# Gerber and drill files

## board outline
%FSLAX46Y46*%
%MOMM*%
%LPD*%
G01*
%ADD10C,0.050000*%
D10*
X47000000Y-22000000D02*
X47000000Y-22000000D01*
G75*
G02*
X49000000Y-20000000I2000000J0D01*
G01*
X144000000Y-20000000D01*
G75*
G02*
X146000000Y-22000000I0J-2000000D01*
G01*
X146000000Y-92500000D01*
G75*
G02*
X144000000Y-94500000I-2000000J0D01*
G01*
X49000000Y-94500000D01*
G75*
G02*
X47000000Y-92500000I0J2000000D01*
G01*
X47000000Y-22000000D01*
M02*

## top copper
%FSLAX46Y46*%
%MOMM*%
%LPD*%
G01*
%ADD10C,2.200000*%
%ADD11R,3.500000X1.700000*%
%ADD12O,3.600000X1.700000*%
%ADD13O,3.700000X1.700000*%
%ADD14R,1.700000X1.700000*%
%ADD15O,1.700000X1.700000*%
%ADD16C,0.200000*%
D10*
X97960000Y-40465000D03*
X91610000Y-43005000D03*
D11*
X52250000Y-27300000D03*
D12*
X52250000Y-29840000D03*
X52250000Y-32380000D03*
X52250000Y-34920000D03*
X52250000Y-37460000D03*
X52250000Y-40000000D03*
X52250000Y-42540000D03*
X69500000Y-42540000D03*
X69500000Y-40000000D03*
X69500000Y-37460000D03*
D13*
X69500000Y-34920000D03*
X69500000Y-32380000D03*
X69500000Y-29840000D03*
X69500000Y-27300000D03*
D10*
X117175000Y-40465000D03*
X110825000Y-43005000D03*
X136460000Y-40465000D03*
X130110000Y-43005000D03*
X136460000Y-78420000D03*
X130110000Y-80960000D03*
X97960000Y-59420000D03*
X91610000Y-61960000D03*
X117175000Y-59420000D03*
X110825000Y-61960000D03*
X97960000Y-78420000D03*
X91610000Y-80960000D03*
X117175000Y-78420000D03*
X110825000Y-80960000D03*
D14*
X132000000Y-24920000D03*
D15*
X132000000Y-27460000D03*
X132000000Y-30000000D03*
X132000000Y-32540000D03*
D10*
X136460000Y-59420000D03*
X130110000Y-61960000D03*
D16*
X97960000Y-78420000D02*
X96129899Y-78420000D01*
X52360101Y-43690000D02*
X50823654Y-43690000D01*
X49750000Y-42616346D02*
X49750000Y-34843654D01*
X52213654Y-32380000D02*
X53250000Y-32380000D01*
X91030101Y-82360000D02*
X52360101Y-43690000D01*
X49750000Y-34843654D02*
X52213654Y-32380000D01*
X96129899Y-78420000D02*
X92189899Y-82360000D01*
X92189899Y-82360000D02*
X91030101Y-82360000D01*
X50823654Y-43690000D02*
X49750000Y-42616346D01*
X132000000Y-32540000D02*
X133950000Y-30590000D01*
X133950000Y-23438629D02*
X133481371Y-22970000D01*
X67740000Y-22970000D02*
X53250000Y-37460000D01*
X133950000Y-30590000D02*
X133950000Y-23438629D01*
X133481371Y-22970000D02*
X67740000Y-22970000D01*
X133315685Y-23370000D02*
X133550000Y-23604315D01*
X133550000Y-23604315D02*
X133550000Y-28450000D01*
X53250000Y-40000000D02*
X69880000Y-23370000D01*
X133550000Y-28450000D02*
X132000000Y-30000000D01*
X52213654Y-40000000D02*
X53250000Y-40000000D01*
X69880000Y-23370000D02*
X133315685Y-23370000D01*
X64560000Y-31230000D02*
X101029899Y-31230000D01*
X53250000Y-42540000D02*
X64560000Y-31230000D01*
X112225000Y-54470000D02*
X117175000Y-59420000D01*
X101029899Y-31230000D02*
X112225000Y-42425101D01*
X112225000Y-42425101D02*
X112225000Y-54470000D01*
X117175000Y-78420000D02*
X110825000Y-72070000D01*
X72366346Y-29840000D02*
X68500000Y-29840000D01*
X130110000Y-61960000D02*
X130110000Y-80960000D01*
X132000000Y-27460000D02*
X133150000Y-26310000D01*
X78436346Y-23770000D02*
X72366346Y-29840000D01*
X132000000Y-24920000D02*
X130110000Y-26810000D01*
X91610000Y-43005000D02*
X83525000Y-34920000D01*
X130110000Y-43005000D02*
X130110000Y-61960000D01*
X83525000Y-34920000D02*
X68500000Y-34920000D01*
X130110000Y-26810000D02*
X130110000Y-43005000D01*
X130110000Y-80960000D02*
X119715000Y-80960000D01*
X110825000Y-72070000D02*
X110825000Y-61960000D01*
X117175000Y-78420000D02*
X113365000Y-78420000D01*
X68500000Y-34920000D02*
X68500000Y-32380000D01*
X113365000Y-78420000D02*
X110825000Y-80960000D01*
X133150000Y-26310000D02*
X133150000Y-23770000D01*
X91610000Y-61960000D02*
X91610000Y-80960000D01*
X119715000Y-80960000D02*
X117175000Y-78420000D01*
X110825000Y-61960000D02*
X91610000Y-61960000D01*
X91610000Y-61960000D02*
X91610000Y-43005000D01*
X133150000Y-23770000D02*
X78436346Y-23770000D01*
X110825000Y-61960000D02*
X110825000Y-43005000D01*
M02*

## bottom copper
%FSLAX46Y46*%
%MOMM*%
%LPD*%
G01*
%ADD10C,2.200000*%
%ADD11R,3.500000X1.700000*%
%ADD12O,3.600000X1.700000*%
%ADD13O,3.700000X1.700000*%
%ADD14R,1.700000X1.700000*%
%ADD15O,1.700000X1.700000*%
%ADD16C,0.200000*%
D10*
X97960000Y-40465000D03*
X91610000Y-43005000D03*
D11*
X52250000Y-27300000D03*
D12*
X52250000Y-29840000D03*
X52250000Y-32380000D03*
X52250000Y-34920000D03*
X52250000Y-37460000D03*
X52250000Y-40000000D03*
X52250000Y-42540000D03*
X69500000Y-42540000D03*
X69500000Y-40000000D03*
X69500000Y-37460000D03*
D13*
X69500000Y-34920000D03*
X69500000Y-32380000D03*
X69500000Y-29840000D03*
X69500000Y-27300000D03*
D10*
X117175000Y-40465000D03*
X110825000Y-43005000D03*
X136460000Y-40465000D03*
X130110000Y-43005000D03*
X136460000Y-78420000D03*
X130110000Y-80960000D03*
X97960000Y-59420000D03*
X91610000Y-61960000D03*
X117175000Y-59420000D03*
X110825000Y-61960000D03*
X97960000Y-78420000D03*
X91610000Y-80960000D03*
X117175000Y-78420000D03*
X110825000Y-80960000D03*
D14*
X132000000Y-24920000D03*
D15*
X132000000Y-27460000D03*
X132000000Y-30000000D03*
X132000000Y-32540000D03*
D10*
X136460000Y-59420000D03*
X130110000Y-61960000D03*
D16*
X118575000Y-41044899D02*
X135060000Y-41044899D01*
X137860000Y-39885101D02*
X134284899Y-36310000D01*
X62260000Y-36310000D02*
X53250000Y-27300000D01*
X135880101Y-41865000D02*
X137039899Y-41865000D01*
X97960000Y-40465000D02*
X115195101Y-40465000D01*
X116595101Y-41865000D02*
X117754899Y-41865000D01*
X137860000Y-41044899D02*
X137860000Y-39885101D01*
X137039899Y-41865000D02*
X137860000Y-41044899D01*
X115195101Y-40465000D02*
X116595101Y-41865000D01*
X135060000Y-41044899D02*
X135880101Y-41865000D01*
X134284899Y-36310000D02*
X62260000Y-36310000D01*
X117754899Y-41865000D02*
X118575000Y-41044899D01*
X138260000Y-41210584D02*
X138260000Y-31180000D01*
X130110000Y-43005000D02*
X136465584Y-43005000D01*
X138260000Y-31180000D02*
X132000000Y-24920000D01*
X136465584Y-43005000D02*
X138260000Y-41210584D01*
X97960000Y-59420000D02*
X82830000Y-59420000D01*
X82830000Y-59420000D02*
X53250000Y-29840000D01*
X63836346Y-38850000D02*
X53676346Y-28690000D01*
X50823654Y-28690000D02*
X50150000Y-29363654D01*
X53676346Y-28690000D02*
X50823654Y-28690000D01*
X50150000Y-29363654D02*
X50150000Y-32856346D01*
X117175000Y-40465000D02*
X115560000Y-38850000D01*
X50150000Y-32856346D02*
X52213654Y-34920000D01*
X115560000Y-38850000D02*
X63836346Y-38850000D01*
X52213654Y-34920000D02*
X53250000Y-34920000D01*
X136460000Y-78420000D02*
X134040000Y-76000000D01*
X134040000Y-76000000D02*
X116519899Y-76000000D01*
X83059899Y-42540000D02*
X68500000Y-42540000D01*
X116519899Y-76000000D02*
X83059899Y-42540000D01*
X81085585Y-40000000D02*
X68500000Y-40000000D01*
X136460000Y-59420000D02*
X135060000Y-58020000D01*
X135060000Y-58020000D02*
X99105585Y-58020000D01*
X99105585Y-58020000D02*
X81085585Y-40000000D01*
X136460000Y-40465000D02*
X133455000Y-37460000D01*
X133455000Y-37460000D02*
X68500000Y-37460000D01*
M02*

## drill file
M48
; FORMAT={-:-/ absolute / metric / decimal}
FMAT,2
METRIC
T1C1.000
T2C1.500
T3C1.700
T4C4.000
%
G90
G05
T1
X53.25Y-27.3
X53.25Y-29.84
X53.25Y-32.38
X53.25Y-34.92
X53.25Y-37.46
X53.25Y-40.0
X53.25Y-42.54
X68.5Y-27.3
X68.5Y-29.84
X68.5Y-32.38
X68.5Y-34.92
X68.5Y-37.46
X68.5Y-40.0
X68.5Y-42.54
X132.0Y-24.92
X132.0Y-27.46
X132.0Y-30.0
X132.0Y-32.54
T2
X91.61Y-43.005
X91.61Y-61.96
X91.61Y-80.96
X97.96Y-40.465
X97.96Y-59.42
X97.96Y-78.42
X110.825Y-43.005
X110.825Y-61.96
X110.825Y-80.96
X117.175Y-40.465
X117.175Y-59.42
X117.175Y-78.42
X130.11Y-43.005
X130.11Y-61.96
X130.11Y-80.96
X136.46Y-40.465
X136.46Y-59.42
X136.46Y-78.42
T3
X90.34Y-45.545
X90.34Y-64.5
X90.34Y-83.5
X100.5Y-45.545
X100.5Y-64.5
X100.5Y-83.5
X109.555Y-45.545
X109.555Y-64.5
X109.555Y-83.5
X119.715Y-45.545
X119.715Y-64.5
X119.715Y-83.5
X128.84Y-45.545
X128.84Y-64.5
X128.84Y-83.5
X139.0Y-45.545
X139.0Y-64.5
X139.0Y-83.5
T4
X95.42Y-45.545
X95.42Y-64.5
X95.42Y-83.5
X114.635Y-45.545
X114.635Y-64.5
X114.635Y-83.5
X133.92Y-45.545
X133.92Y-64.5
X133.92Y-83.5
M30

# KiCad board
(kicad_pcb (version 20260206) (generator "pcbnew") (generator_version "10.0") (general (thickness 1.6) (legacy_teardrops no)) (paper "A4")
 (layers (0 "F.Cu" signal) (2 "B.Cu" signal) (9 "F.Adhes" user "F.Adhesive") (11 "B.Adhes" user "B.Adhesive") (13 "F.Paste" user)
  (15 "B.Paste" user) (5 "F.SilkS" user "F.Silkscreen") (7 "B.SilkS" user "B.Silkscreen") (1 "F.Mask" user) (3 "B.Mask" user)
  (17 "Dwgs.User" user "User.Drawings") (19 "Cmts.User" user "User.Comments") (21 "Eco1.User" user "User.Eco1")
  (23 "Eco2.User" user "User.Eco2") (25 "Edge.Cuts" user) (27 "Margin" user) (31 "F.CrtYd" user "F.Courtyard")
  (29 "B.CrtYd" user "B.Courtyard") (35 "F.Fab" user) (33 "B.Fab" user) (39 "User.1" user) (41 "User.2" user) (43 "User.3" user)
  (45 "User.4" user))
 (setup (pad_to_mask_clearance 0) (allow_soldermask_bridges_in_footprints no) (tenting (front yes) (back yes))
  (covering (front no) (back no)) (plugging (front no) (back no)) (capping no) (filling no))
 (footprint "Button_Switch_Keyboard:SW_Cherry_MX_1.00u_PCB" (layer "F.Cu") (at 97.96 40.465)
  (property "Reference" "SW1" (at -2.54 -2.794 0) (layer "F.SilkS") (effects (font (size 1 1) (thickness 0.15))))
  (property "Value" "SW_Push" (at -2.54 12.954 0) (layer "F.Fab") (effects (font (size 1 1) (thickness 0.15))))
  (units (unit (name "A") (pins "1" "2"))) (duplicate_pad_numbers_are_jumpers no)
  (pad "" np_thru_hole circle (at -7.62 5.08) (size 1.7 1.7) (drill 1.7) (layers "*.Cu" "*.Mask"))
  (pad "" np_thru_hole circle (at -2.54 5.08) (size 4 4) (drill 4) (layers "*.Cu" "*.Mask"))
  (pad "" np_thru_hole circle (at 2.54 5.08) (size 1.7 1.7) (drill 1.7) (layers "*.Cu" "*.Mask"))
  (pad "1" thru_hole circle (at 0 0) (size 2.2 2.2) (drill 1.5) (layers "*.Cu" "*.Mask") (remove_unused_layers no) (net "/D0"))
  (pad "2" thru_hole circle (at -6.35 2.54) (size 2.2 2.2) (drill 1.5) (layers "*.Cu" "*.Mask") (remove_unused_layers no) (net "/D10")))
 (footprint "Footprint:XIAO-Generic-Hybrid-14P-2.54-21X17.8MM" (layer "F.Cu") (at 60.875 34.92)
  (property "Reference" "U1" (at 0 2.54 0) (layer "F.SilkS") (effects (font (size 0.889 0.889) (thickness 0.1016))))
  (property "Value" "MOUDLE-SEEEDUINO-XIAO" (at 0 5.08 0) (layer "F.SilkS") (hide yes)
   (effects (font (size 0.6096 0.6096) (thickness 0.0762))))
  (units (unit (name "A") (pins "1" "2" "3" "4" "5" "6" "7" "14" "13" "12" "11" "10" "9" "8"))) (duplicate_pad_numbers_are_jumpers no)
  (pad "1" thru_hole rect (at -7.625 -7.62) (size 3.5 1.7) (drill 1 (offset -1 0)) (layers "*.Cu" "*.Mask") (remove_unused_layers no)
   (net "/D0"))
  (pad "2" thru_hole oval (at -7.625 -5.08) (size 3.6 1.7) (drill 1 (offset -1 0)) (layers "*.Cu" "*.Mask") (remove_unused_layers no)
   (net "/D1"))
  (pad "3" thru_hole oval (at -7.625 -2.54) (size 3.6 1.7) (drill 1 (offset -1 0)) (layers "*.Cu" "*.Mask") (remove_unused_layers no)
   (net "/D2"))
  (pad "4" thru_hole oval (at -7.625 0) (size 3.6 1.7) (drill 1 (offset -1 0)) (layers "*.Cu" "*.Mask") (remove_unused_layers no)
   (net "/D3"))
  (pad "5" thru_hole oval (at -7.625 2.54) (size 3.6 1.7) (drill 1 (offset -1 0)) (layers "*.Cu" "*.Mask") (remove_unused_layers no)
   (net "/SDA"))
  (pad "6" thru_hole oval (at -7.625 5.08 180) (size 3.6 1.7) (drill 1 (offset 1 0)) (layers "*.Cu" "*.Mask") (remove_unused_layers no)
   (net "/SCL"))
  (pad "7" thru_hole oval (at -7.625 7.62) (size 3.6 1.7) (drill 1 (offset -1 0)) (layers "*.Cu" "*.Mask") (remove_unused_layers no)
   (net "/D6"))
  (pad "8" thru_hole oval (at 7.625 7.62) (size 3.6 1.7) (drill 1 (offset 1 0)) (layers "*.Cu" "*.Mask") (remove_unused_layers no)
   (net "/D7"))
  (pad "9" thru_hole oval (at 7.625 5.08) (size 3.6 1.7) (drill 1 (offset 1 0)) (layers "*.Cu" "*.Mask") (remove_unused_layers no)
   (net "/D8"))
  (pad "10" thru_hole oval (at 7.625 2.54) (size 3.6 1.7) (drill 1 (offset 1 0)) (layers "*.Cu" "*.Mask") (remove_unused_layers no)
   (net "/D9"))
  (pad "11" thru_hole oval (at 7.625 0) (size 3.7 1.7) (drill 1 (offset 1 0)) (layers "*.Cu" "*.Mask") (remove_unused_layers no)
   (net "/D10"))
  (pad "12" thru_hole oval (at 7.625 -2.54) (size 3.7 1.7) (drill 1 (offset 1 0)) (layers "*.Cu" "*.Mask") (remove_unused_layers no)
   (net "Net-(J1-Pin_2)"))
  (pad "13" thru_hole oval (at 7.625 -5.08) (size 3.7 1.7) (drill 1 (offset 1 0)) (layers "*.Cu" "*.Mask") (remove_unused_layers no)
   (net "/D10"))
  (pad "14" thru_hole oval (at 7.625 -7.62) (size 3.7 1.7) (drill 1 (offset 1 0)) (layers "*.Cu" "*.Mask") (remove_unused_layers no)
   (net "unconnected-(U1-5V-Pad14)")))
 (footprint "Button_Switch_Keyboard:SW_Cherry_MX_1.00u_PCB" (layer "F.Cu") (at 117.175 40.465)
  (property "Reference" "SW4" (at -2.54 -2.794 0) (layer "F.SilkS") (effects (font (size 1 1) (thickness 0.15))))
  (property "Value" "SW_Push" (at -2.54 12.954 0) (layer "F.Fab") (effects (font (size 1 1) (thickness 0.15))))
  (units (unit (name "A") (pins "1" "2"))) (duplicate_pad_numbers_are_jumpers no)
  (pad "" np_thru_hole circle (at -7.62 5.08) (size 1.7 1.7) (drill 1.7) (layers "*.Cu" "*.Mask"))
  (pad "" np_thru_hole circle (at -2.54 5.08) (size 4 4) (drill 4) (layers "*.Cu" "*.Mask"))
  (pad "" np_thru_hole circle (at 2.54 5.08) (size 1.7 1.7) (drill 1.7) (layers "*.Cu" "*.Mask"))
  (pad "1" thru_hole circle (at 0 0) (size 2.2 2.2) (drill 1.5) (layers "*.Cu" "*.Mask") (remove_unused_layers no) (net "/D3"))
  (pad "2" thru_hole circle (at -6.35 2.54) (size 2.2 2.2) (drill 1.5) (layers "*.Cu" "*.Mask") (remove_unused_layers no) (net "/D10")))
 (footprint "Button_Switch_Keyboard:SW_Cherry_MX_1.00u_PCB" (layer "F.Cu") (at 136.46 40.465)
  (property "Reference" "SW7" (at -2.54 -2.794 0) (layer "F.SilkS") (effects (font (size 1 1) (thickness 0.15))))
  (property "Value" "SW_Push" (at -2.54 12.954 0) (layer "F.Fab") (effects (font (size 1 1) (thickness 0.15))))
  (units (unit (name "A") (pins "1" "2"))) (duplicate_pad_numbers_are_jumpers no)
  (pad "" np_thru_hole circle (at -7.62 5.08) (size 1.7 1.7) (drill 1.7) (layers "*.Cu" "*.Mask"))
  (pad "" np_thru_hole circle (at -2.54 5.08) (size 4 4) (drill 4) (layers "*.Cu" "*.Mask"))
  (pad "" np_thru_hole circle (at 2.54 5.08) (size 1.7 1.7) (drill 1.7) (layers "*.Cu" "*.Mask"))
  (pad "1" thru_hole circle (at 0 0) (size 2.2 2.2) (drill 1.5) (layers "*.Cu" "*.Mask") (remove_unused_layers no) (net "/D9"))
  (pad "2" thru_hole circle (at -6.35 2.54) (size 2.2 2.2) (drill 1.5) (layers "*.Cu" "*.Mask") (remove_unused_layers no) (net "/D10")))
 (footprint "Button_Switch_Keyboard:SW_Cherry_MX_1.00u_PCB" (layer "F.Cu") (at 136.46 78.42)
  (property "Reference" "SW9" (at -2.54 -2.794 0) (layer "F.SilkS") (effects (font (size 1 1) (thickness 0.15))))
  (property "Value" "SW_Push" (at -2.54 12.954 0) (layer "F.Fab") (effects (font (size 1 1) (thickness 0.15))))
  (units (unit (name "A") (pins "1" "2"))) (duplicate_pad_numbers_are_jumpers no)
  (pad "" np_thru_hole circle (at -7.62 5.08) (size 1.7 1.7) (drill 1.7) (layers "*.Cu" "*.Mask"))
  (pad "" np_thru_hole circle (at -2.54 5.08) (size 4 4) (drill 4) (layers "*.Cu" "*.Mask"))
  (pad "" np_thru_hole circle (at 2.54 5.08) (size 1.7 1.7) (drill 1.7) (layers "*.Cu" "*.Mask"))
  (pad "1" thru_hole circle (at 0 0) (size 2.2 2.2) (drill 1.5) (layers "*.Cu" "*.Mask") (remove_unused_layers no) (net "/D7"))
  (pad "2" thru_hole circle (at -6.35 2.54) (size 2.2 2.2) (drill 1.5) (layers "*.Cu" "*.Mask") (remove_unused_layers no) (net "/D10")))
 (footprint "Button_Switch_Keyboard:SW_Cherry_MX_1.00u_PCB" (layer "F.Cu") (at 97.96 59.42)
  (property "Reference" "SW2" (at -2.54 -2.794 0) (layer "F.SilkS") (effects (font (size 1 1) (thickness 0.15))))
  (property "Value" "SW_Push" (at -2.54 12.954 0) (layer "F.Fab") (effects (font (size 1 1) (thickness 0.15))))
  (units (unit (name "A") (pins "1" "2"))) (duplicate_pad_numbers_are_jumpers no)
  (pad "" np_thru_hole circle (at -7.62 5.08) (size 1.7 1.7) (drill 1.7) (layers "*.Cu" "*.Mask"))
  (pad "" np_thru_hole circle (at -2.54 5.08) (size 4 4) (drill 4) (layers "*.Cu" "*.Mask"))
  (pad "" np_thru_hole circle (at 2.54 5.08) (size 1.7 1.7) (drill 1.7) (layers "*.Cu" "*.Mask"))
  (pad "1" thru_hole circle (at 0 0) (size 2.2 2.2) (drill 1.5) (layers "*.Cu" "*.Mask") (remove_unused_layers no) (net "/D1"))
  (pad "2" thru_hole circle (at -6.35 2.54) (size 2.2 2.2) (drill 1.5) (layers "*.Cu" "*.Mask") (remove_unused_layers no) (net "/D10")))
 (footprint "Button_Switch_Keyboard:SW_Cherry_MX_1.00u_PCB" (layer "F.Cu") (at 117.175 59.42)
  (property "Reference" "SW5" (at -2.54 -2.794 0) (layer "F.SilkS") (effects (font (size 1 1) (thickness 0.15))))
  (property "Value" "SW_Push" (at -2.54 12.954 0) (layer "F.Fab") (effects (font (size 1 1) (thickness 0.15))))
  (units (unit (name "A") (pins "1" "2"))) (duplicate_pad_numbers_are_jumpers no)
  (pad "" np_thru_hole circle (at -7.62 5.08) (size 1.7 1.7) (drill 1.7) (layers "*.Cu" "*.Mask"))
  (pad "" np_thru_hole circle (at -2.54 5.08) (size 4 4) (drill 4) (layers "*.Cu" "*.Mask"))
  (pad "" np_thru_hole circle (at 2.54 5.08) (size 1.7 1.7) (drill 1.7) (layers "*.Cu" "*.Mask"))
  (pad "1" thru_hole circle (at 0 0) (size 2.2 2.2) (drill 1.5) (layers "*.Cu" "*.Mask") (remove_unused_layers no) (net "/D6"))
  (pad "2" thru_hole circle (at -6.35 2.54) (size 2.2 2.2) (drill 1.5) (layers "*.Cu" "*.Mask") (remove_unused_layers no) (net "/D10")))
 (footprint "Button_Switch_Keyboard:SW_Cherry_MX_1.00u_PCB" (layer "F.Cu") (at 97.96 78.42)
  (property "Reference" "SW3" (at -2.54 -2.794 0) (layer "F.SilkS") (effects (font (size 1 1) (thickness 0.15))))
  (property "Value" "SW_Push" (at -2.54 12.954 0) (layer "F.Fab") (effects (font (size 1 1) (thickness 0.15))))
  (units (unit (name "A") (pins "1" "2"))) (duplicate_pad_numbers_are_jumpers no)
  (pad "" np_thru_hole circle (at -7.62 5.08) (size 1.7 1.7) (drill 1.7) (layers "*.Cu" "*.Mask"))
  (pad "" np_thru_hole circle (at -2.54 5.08) (size 4 4) (drill 4) (layers "*.Cu" "*.Mask"))
  (pad "" np_thru_hole circle (at 2.54 5.08) (size 1.7 1.7) (drill 1.7) (layers "*.Cu" "*.Mask"))
  (pad "1" thru_hole circle (at 0 0) (size 2.2 2.2) (drill 1.5) (layers "*.Cu" "*.Mask") (remove_unused_layers no) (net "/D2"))
  (pad "2" thru_hole circle (at -6.35 2.54) (size 2.2 2.2) (drill 1.5) (layers "*.Cu" "*.Mask") (remove_unused_layers no) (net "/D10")))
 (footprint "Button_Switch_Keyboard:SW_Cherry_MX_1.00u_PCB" (layer "F.Cu") (at 117.175 78.42)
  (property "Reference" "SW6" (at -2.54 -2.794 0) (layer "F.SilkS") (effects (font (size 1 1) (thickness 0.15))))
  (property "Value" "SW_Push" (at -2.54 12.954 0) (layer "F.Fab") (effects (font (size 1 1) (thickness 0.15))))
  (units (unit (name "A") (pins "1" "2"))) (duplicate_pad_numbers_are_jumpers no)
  (pad "" np_thru_hole circle (at -7.62 5.08) (size 1.7 1.7) (drill 1.7) (layers "*.Cu" "*.Mask"))
  (pad "" np_thru_hole circle (at -2.54 5.08) (size 4 4) (drill 4) (layers "*.Cu" "*.Mask"))
  (pad "" np_thru_hole circle (at 2.54 5.08) (size 1.7 1.7) (drill 1.7) (layers "*.Cu" "*.Mask"))
  (pad "1" thru_hole circle (at 0 0) (size 2.2 2.2) (drill 1.5) (layers "*.Cu" "*.Mask") (remove_unused_layers no) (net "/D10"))
  (pad "2" thru_hole circle (at -6.35 2.54) (size 2.2 2.2) (drill 1.5) (layers "*.Cu" "*.Mask") (remove_unused_layers no) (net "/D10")))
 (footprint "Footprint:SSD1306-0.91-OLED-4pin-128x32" (layer "F.Cu") (at 95.5 22.73)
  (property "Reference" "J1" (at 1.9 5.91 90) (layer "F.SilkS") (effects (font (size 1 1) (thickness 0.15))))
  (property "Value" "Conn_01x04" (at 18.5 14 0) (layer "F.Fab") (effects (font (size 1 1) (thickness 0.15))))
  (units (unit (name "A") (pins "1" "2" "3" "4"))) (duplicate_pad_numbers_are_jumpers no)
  (pad "1" thru_hole rect (at 36.5 2.19) (size 1.7 1.7) (drill 1) (layers "*.Cu" "*.Mask") (remove_unused_layers no) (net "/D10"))
  (pad "2" thru_hole oval (at 36.5 4.73) (size 1.7 1.7) (drill 1) (layers "*.Cu" "*.Mask") (remove_unused_layers no) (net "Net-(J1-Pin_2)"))
  (pad "3" thru_hole oval (at 36.5 7.27) (size 1.7 1.7) (drill 1) (layers "*.Cu" "*.Mask") (remove_unused_layers no) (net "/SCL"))
  (pad "4" thru_hole oval (at 36.5 9.81) (size 1.7 1.7) (drill 1) (layers "*.Cu" "*.Mask") (remove_unused_layers no) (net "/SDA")))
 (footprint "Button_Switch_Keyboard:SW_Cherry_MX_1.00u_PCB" (layer "F.Cu") (at 136.46 59.42)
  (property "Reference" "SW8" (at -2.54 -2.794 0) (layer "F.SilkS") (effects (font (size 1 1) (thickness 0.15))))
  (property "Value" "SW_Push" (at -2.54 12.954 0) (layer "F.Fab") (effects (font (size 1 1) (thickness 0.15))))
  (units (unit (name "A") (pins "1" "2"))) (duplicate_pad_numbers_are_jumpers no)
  (pad "" np_thru_hole circle (at -7.62 5.08) (size 1.7 1.7) (drill 1.7) (layers "*.Cu" "*.Mask"))
  (pad "" np_thru_hole circle (at -2.54 5.08) (size 4 4) (drill 4) (layers "*.Cu" "*.Mask"))
  (pad "" np_thru_hole circle (at 2.54 5.08) (size 1.7 1.7) (drill 1.7) (layers "*.Cu" "*.Mask"))
  (pad "1" thru_hole circle (at 0 0) (size 2.2 2.2) (drill 1.5) (layers "*.Cu" "*.Mask") (remove_unused_layers no) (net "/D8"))
  (pad "2" thru_hole circle (at -6.35 2.54) (size 2.2 2.2) (drill 1.5) (layers "*.Cu" "*.Mask") (remove_unused_layers no) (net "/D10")))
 (gr_rect (start 47 20) (end 146 94.5) (radius 2) (stroke (width 0.05) (type solid)) (fill no) (layer "Edge.Cuts"))
 (segment (start 118.575 41.044899) (end 135.06 41.044899) (width 0.2) (layer "B.Cu") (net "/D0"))
 (segment (start 137.86 39.885101) (end 134.284899 36.31) (width 0.2) (layer "B.Cu") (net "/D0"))
 (segment (start 62.26 36.31) (end 53.25 27.3) (width 0.2) (layer "B.Cu") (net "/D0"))
 (segment (start 135.880101 41.865) (end 137.039899 41.865) (width 0.2) (layer "B.Cu") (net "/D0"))
 (segment (start 97.96 40.465) (end 115.195101 40.465) (width 0.2) (layer "B.Cu") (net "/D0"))
 (segment (start 116.595101 41.865) (end 117.754899 41.865) (width 0.2) (layer "B.Cu") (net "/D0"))
 (segment (start 137.86 41.044899) (end 137.86 39.885101) (width 0.2) (layer "B.Cu") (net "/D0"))
 (segment (start 137.039899 41.865) (end 137.86 41.044899) (width 0.2) (layer "B.Cu") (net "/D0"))
 (segment (start 115.195101 40.465) (end 116.595101 41.865) (width 0.2) (layer "B.Cu") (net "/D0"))
 (segment (start 135.06 41.044899) (end 135.880101 41.865) (width 0.2) (layer "B.Cu") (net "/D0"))
 (segment (start 134.284899 36.31) (end 62.26 36.31) (width 0.2) (layer "B.Cu") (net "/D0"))
 (segment (start 117.754899 41.865) (end 118.575 41.044899) (width 0.2) (layer "B.Cu") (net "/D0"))
 (segment (start 138.26 41.210584) (end 138.26 31.18) (width 0.2) (layer "B.Cu") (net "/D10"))
 (segment (start 130.11 43.005) (end 136.465584 43.005) (width 0.2) (layer "B.Cu") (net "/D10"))
 (segment (start 138.26 31.18) (end 132 24.92) (width 0.2) (layer "B.Cu") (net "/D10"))
 (segment (start 136.465584 43.005) (end 138.26 41.210584) (width 0.2) (layer "B.Cu") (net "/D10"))
 (segment (start 97.96 59.42) (end 82.83 59.42) (width 0.2) (layer "B.Cu") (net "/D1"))
 (segment (start 82.83 59.42) (end 53.25 29.84) (width 0.2) (layer "B.Cu") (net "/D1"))
 (segment (start 97.96 78.42) (end 96.129899 78.42) (width 0.2) (layer "F.Cu") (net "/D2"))
 (segment (start 52.360101 43.69) (end 50.823654 43.69) (width 0.2) (layer "F.Cu") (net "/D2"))
 (segment (start 49.75 42.616346) (end 49.75 34.843654) (width 0.2) (layer "F.Cu") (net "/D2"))
 (segment (start 52.213654 32.38) (end 53.25 32.38) (width 0.2) (layer "F.Cu") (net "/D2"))
 (segment (start 91.030101 82.36) (end 52.360101 43.69) (width 0.2) (layer "F.Cu") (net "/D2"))
 (segment (start 49.75 34.843654) (end 52.213654 32.38) (width 0.2) (layer "F.Cu") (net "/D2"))
 (segment (start 96.129899 78.42) (end 92.189899 82.36) (width 0.2) (layer "F.Cu") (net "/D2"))
 (segment (start 92.189899 82.36) (end 91.030101 82.36) (width 0.2) (layer "F.Cu") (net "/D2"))
 (segment (start 50.823654 43.69) (end 49.75 42.616346) (width 0.2) (layer "F.Cu") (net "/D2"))
 (segment (start 63.836346 38.85) (end 53.676346 28.69) (width 0.2) (layer "B.Cu") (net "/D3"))
 (segment (start 50.823654 28.69) (end 50.15 29.363654) (width 0.2) (layer "B.Cu") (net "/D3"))
 (segment (start 53.676346 28.69) (end 50.823654 28.69) (width 0.2) (layer "B.Cu") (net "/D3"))
 (segment (start 50.15 29.363654) (end 50.15 32.856346) (width 0.2) (layer "B.Cu") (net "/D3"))
 (segment (start 117.175 40.465) (end 115.56 38.85) (width 0.2) (layer "B.Cu") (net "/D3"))
 (segment (start 50.15 32.856346) (end 52.213654 34.92) (width 0.2) (layer "B.Cu") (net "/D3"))
 (segment (start 115.56 38.85) (end 63.836346 38.85) (width 0.2) (layer "B.Cu") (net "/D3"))
 (segment (start 52.213654 34.92) (end 53.25 34.92) (width 0.2) (layer "B.Cu") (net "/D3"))
 (segment (start 132 32.54) (end 133.95 30.59) (width 0.2) (layer "F.Cu") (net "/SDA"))
 (segment (start 133.95 23.438629) (end 133.481371 22.97) (width 0.2) (layer "F.Cu") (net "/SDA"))
 (segment (start 67.74 22.97) (end 53.25 37.46) (width 0.2) (layer "F.Cu") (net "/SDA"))
 (segment (start 133.95 30.59) (end 133.95 23.438629) (width 0.2) (layer "F.Cu") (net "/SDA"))
 (segment (start 133.481371 22.97) (end 67.74 22.97) (width 0.2) (layer "F.Cu") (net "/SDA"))
 (segment (start 133.315685 23.37) (end 133.55 23.604315) (width 0.2) (layer "F.Cu") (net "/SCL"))
 (segment (start 133.55 23.604315) (end 133.55 28.45) (width 0.2) (layer "F.Cu") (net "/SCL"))
 (segment (start 53.25 40) (end 69.88 23.37) (width 0.2) (layer "F.Cu") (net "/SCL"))
 (segment (start 133.55 28.45) (end 132 30) (width 0.2) (layer "F.Cu") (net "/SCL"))
 (segment (start 52.213654 40) (end 53.25 40) (width 0.2) (layer "F.Cu") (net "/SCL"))
 (segment (start 69.88 23.37) (end 133.315685 23.37) (width 0.2) (layer "F.Cu") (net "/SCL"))
 (segment (start 64.56 31.23) (end 101.029899 31.23) (width 0.2) (layer "F.Cu") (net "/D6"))
 (segment (start 53.25 42.54) (end 64.56 31.23) (width 0.2) (layer "F.Cu") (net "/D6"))
 (segment (start 112.225 54.47) (end 117.175 59.42) (width 0.2) (layer "F.Cu") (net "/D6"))
 (segment (start 101.029899 31.23) (end 112.225 42.425101) (width 0.2) (layer "F.Cu") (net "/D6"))
 (segment (start 112.225 42.425101) (end 112.225 54.47) (width 0.2) (layer "F.Cu") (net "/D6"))
 (segment (start 136.46 78.42) (end 134.04 76) (width 0.2) (layer "B.Cu") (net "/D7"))
 (segment (start 134.04 76) (end 116.519899 76) (width 0.2) (layer "B.Cu") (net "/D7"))
 (segment (start 83.059899 42.54) (end 68.5 42.54) (width 0.2) (layer "B.Cu") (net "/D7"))
 (segment (start 116.519899 76) (end 83.059899 42.54) (width 0.2) (layer "B.Cu") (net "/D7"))
 (segment (start 81.085585 40) (end 68.5 40) (width 0.2) (layer "B.Cu") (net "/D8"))
 (segment (start 136.46 59.42) (end 135.06 58.02) (width 0.2) (layer "B.Cu") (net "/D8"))
 (segment (start 135.06 58.02) (end 99.105585 58.02) (width 0.2) (layer "B.Cu") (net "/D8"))
 (segment (start 99.105585 58.02) (end 81.085585 40) (width 0.2) (layer "B.Cu") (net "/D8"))
 (segment (start 136.46 40.465) (end 133.455 37.46) (width 0.2) (layer "B.Cu") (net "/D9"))
 (segment (start 133.455 37.46) (end 68.5 37.46) (width 0.2) (layer "B.Cu") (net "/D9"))
 (segment (start 117.175 78.42) (end 110.825 72.07) (width 0.2) (layer "F.Cu") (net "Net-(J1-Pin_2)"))
 (segment (start 72.366346 29.84) (end 68.5 29.84) (width 0.2) (layer "F.Cu") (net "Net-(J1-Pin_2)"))
 (segment (start 130.11 61.96) (end 130.11 80.96) (width 0.2) (layer "F.Cu") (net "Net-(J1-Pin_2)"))
 (segment (start 132 27.46) (end 133.15 26.31) (width 0.2) (layer "F.Cu") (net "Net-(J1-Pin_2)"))
 (segment (start 78.436346 23.77) (end 72.366346 29.84) (width 0.2) (layer "F.Cu") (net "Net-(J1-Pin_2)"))
 (segment (start 132 24.92) (end 130.11 26.81) (width 0.2) (layer "F.Cu") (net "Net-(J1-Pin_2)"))
 (segment (start 91.61 43.005) (end 83.525 34.92) (width 0.2) (layer "F.Cu") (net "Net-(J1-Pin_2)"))
 (segment (start 130.11 43.005) (end 130.11 61.96) (width 0.2) (layer "F.Cu") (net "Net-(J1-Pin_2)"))
 (segment (start 83.525 34.92) (end 68.5 34.92) (width 0.2) (layer "F.Cu") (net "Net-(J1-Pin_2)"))
 (segment (start 130.11 26.81) (end 130.11 43.005) (width 0.2) (layer "F.Cu") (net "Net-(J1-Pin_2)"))
 (segment (start 130.11 80.96) (end 119.715 80.96) (width 0.2) (layer "F.Cu") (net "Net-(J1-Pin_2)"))
 (segment (start 110.825 72.07) (end 110.825 61.96) (width 0.2) (layer "F.Cu") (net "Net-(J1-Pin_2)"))
 (segment (start 117.175 78.42) (end 113.365 78.42) (width 0.2) (layer "F.Cu") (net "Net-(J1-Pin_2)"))
 (segment (start 68.5 34.92) (end 68.5 32.38) (width 0.2) (layer "F.Cu") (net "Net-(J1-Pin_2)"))
 (segment (start 113.365 78.42) (end 110.825 80.96) (width 0.2) (layer "F.Cu") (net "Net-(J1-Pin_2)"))
 (segment (start 133.15 26.31) (end 133.15 23.77) (width 0.2) (layer "F.Cu") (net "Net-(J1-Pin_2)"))
 (segment (start 91.61 61.96) (end 91.61 80.96) (width 0.2) (layer "F.Cu") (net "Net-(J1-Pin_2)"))
 (segment (start 119.715 80.96) (end 117.175 78.42) (width 0.2) (layer "F.Cu") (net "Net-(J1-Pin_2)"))
 (segment (start 110.825 61.96) (end 91.61 61.96) (width 0.2) (layer "F.Cu") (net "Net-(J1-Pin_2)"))
 (segment (start 91.61 61.96) (end 91.61 43.005) (width 0.2) (layer "F.Cu") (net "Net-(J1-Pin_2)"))
 (segment (start 133.15 23.77) (end 78.436346 23.77) (width 0.2) (layer "F.Cu") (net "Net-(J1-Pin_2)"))
 (segment (start 110.825 61.96) (end 110.825 43.005) (width 0.2) (layer "F.Cu") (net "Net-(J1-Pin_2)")))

